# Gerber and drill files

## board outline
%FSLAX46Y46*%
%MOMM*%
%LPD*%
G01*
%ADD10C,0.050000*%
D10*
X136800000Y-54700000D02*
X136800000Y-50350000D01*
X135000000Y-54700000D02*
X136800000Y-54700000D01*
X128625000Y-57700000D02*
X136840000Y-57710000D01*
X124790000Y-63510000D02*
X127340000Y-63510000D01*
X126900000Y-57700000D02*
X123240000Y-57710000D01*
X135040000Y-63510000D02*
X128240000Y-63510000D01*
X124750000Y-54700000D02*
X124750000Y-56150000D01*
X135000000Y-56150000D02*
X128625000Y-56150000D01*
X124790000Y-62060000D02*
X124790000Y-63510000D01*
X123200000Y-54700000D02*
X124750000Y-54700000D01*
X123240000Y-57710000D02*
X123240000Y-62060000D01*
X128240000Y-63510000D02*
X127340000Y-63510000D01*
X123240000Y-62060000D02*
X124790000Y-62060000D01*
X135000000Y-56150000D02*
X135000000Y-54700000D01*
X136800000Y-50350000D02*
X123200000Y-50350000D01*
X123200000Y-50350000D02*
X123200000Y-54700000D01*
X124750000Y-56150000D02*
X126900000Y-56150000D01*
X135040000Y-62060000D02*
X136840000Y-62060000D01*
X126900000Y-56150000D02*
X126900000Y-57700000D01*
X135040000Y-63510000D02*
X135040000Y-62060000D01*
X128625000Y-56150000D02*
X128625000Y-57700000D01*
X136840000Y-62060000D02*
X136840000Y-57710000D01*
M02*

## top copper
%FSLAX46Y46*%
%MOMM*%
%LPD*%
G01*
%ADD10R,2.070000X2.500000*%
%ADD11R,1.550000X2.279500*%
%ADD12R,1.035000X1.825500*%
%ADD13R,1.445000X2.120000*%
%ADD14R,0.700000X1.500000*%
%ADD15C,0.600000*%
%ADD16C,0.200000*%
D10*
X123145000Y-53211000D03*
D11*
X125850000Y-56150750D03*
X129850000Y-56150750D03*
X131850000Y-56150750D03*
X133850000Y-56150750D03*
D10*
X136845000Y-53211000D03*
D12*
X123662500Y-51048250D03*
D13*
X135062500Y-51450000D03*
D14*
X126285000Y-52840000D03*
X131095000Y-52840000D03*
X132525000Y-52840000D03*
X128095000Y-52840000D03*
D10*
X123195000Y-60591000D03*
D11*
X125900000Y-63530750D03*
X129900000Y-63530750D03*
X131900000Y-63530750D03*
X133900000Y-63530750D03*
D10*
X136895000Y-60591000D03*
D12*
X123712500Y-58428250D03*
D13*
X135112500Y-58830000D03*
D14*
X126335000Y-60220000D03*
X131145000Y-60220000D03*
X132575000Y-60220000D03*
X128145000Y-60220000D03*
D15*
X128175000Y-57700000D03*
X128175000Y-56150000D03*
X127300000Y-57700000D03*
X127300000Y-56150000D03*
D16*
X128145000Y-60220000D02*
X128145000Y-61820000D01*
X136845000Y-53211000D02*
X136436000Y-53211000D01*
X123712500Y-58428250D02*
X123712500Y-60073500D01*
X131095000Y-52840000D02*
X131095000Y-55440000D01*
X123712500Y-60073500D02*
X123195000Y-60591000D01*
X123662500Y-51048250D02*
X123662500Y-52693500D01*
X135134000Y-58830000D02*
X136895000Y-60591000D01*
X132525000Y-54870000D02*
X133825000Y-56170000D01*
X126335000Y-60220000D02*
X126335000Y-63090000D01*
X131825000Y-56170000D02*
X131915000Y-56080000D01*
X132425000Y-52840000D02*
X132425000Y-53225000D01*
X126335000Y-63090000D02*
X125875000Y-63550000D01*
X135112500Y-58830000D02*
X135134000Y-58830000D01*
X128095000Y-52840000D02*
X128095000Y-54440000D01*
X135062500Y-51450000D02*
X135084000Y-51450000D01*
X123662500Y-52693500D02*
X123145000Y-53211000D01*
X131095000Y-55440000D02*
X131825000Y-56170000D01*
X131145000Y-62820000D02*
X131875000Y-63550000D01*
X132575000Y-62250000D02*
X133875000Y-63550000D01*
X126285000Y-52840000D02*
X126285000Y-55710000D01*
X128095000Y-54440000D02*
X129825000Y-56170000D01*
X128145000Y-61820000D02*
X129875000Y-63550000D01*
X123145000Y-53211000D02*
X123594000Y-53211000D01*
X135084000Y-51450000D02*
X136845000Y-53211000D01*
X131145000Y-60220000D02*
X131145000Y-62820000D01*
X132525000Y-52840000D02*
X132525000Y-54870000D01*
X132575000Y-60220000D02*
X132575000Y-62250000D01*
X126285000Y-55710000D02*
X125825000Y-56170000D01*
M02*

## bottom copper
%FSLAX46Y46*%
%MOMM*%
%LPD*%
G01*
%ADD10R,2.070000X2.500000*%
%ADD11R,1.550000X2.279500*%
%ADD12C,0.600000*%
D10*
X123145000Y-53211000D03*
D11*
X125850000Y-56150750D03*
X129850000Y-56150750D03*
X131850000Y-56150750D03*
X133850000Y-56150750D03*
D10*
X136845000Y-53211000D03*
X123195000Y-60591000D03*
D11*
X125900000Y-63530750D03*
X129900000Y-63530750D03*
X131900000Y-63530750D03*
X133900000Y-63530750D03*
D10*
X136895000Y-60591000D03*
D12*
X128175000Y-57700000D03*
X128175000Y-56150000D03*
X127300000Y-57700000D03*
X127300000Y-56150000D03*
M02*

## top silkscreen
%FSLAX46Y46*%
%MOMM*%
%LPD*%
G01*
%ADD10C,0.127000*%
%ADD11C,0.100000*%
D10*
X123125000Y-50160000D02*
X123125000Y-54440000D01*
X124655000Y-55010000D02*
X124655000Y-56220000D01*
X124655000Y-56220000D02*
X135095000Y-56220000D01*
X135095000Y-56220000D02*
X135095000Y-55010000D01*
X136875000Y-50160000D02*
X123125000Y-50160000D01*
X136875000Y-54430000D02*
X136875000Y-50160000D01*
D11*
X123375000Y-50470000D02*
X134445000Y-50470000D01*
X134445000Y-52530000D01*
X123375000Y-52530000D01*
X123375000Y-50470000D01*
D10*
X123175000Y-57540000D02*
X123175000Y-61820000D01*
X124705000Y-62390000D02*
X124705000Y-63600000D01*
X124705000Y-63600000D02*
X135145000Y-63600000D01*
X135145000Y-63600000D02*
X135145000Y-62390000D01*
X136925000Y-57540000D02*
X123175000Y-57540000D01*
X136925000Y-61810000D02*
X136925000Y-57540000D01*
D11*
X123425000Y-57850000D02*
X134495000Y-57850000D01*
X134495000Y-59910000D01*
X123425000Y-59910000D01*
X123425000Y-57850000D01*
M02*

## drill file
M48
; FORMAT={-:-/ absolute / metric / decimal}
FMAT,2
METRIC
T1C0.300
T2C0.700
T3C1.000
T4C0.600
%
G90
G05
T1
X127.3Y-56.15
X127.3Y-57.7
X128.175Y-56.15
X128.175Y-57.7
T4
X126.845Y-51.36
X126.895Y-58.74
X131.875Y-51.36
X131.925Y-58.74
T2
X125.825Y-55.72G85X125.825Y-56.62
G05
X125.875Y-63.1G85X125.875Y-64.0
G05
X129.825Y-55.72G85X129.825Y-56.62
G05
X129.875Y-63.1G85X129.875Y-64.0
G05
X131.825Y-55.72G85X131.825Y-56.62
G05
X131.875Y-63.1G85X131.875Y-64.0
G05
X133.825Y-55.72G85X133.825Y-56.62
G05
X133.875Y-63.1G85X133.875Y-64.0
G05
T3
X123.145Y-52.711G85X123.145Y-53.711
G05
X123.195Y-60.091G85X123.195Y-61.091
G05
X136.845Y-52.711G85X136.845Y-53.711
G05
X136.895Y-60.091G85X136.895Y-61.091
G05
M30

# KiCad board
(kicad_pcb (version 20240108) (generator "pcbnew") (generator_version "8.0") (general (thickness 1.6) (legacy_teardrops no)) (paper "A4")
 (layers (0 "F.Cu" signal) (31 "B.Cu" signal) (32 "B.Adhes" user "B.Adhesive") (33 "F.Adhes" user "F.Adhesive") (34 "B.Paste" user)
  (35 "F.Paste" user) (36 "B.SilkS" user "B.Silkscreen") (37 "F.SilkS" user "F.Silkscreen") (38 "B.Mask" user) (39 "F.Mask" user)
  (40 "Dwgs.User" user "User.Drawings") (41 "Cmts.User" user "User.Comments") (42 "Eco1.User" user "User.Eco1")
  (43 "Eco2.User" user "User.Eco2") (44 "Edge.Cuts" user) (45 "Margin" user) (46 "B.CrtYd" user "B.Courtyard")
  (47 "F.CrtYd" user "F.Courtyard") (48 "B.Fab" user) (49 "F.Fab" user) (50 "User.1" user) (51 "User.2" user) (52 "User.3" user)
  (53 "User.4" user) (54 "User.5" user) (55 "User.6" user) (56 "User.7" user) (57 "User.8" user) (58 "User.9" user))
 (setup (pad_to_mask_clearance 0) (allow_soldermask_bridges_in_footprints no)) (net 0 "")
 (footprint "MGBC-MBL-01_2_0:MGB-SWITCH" (layer "F.Cu") (at 129.625 53.97)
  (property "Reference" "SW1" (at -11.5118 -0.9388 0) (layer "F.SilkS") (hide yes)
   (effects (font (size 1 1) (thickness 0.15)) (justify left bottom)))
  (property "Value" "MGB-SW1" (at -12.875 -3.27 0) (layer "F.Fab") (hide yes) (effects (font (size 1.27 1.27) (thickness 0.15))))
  (fp_line (start -6.5 -3.81) (end -6.5 0.47) (stroke (width 0.127) (type solid)) (layer "F.SilkS"))
  (fp_line (start -4.97 1.04) (end -4.97 2.25) (stroke (width 0.127) (type solid)) (layer "F.SilkS"))
  (fp_line (start -4.97 2.25) (end 5.47 2.25) (stroke (width 0.127) (type solid)) (layer "F.SilkS"))
  (fp_line (start 5.47 2.25) (end 5.47 1.04) (stroke (width 0.127) (type solid)) (layer "F.SilkS"))
  (fp_line (start 7.25 -3.81) (end -6.5 -3.81) (stroke (width 0.127) (type solid)) (layer "F.SilkS"))
  (fp_line (start 7.25 0.46) (end 7.25 -3.81) (stroke (width 0.127) (type solid)) (layer "F.SilkS"))
  (fp_rect (start -6.25 -3.5) (end 4.82 -1.44) (stroke (width 0.1) (type default)) (fill none) (layer "F.SilkS"))
  (pad "" np_thru_hole circle (at -2.78 -2.61) (size 0.6 0.6) (drill 0.6) (layers "F&B.Cu" "*.Mask"))
  (pad "" np_thru_hole circle (at 2.25 -2.61) (size 0.6 0.6) (drill 0.6) (layers "F&B.Cu" "*.Mask"))
  (pad "1" thru_hole rect (at -6.48 -0.759) (size 2.07 2.5) (drill oval 1 2) (layers "*.Cu" "*.Mask") (remove_unused_layers no))
  (pad "1" thru_hole rect (at -3.8 2.2) (size 1.55 2.2795) (drill oval 0.7 1.6 (offset 0.025 -0.01925)) (layers "*.Cu" "*.Mask")
   (remove_unused_layers no))
  (pad "1" thru_hole rect (at 0.2 2.2) (size 1.55 2.2795) (drill oval 0.7 1.6 (offset 0.025 -0.01925)) (layers "*.Cu" "*.Mask")
   (remove_unused_layers no))
  (pad "1" thru_hole rect (at 2.2 2.2) (size 1.55 2.2795) (drill oval 0.7 1.6 (offset 0.025 -0.01925)) (layers "*.Cu" "*.Mask")
   (remove_unused_layers no))
  (pad "1" thru_hole rect (at 4.2 2.2) (size 1.55 2.2795) (drill oval 0.7 1.6 (offset 0.025 -0.01925)) (layers "*.Cu" "*.Mask")
   (remove_unused_layers no))
  (pad "1" thru_hole rect (at 7.22 -0.759) (size 2.07 2.5) (drill oval 1 2) (layers "*.Cu" "*.Mask") (remove_unused_layers no))
  (pad "2" smd rect (at -5.9625 -2.92175) (size 1.035 1.8255) (layers "F.Cu" "F.Paste" "F.Mask"))
  (pad "3" smd rect (at 5.4375 -2.52) (size 1.445 2.12) (layers "F.Cu" "F.Paste" "F.Mask"))
  (pad "4" smd rect (at -3.34 -1.13) (size 0.7 1.5) (layers "F.Cu" "F.Paste" "F.Mask"))
  (pad "5" smd rect (at 1.47 -1.13) (size 0.7 1.5) (layers "F.Cu" "F.Paste" "F.Mask"))
  (pad "6" smd rect (at 2.9 -1.13) (size 0.7 1.5) (layers "F.Cu" "F.Paste" "F.Mask"))
  (pad "7" smd rect (at -1.53 -1.13) (size 0.7 1.5) (layers "F.Cu" "F.Paste" "F.Mask")))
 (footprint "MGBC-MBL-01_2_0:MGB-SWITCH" (layer "F.Cu") (at 129.675 61.35)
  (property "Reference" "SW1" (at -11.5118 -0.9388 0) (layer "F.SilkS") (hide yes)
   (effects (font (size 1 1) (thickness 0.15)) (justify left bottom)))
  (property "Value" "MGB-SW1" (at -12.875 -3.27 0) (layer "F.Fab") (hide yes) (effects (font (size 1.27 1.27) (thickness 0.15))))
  (fp_line (start -6.5 -3.81) (end -6.5 0.47) (stroke (width 0.127) (type solid)) (layer "F.SilkS"))
  (fp_line (start -4.97 1.04) (end -4.97 2.25) (stroke (width 0.127) (type solid)) (layer "F.SilkS"))
  (fp_line (start -4.97 2.25) (end 5.47 2.25) (stroke (width 0.127) (type solid)) (layer "F.SilkS"))
  (fp_line (start 5.47 2.25) (end 5.47 1.04) (stroke (width 0.127) (type solid)) (layer "F.SilkS"))
  (fp_line (start 7.25 -3.81) (end -6.5 -3.81) (stroke (width 0.127) (type solid)) (layer "F.SilkS"))
  (fp_line (start 7.25 0.46) (end 7.25 -3.81) (stroke (width 0.127) (type solid)) (layer "F.SilkS"))
  (fp_rect (start -6.25 -3.5) (end 4.82 -1.44) (stroke (width 0.1) (type default)) (fill none) (layer "F.SilkS"))
  (pad "" np_thru_hole circle (at -2.78 -2.61) (size 0.6 0.6) (drill 0.6) (layers "F&B.Cu" "*.Mask"))
  (pad "" np_thru_hole circle (at 2.25 -2.61) (size 0.6 0.6) (drill 0.6) (layers "F&B.Cu" "*.Mask"))
  (pad "1" thru_hole rect (at -6.48 -0.759) (size 2.07 2.5) (drill oval 1 2) (layers "*.Cu" "*.Mask") (remove_unused_layers no))
  (pad "1" thru_hole rect (at -3.8 2.2) (size 1.55 2.2795) (drill oval 0.7 1.6 (offset 0.025 -0.01925)) (layers "*.Cu" "*.Mask")
   (remove_unused_layers no))
  (pad "1" thru_hole rect (at 0.2 2.2) (size 1.55 2.2795) (drill oval 0.7 1.6 (offset 0.025 -0.01925)) (layers "*.Cu" "*.Mask")
   (remove_unused_layers no))
  (pad "1" thru_hole rect (at 2.2 2.2) (size 1.55 2.2795) (drill oval 0.7 1.6 (offset 0.025 -0.01925)) (layers "*.Cu" "*.Mask")
   (remove_unused_layers no))
  (pad "1" thru_hole rect (at 4.2 2.2) (size 1.55 2.2795) (drill oval 0.7 1.6 (offset 0.025 -0.01925)) (layers "*.Cu" "*.Mask")
   (remove_unused_layers no))
  (pad "1" thru_hole rect (at 7.22 -0.759) (size 2.07 2.5) (drill oval 1 2) (layers "*.Cu" "*.Mask") (remove_unused_layers no))
  (pad "2" smd rect (at -5.9625 -2.92175) (size 1.035 1.8255) (layers "F.Cu" "F.Paste" "F.Mask"))
  (pad "3" smd rect (at 5.4375 -2.52) (size 1.445 2.12) (layers "F.Cu" "F.Paste" "F.Mask"))
  (pad "4" smd rect (at -3.34 -1.13) (size 0.7 1.5) (layers "F.Cu" "F.Paste" "F.Mask"))
  (pad "5" smd rect (at 1.47 -1.13) (size 0.7 1.5) (layers "F.Cu" "F.Paste" "F.Mask"))
  (pad "6" smd rect (at 2.9 -1.13) (size 0.7 1.5) (layers "F.Cu" "F.Paste" "F.Mask"))
  (pad "7" smd rect (at -1.53 -1.13) (size 0.7 1.5) (layers "F.Cu" "F.Paste" "F.Mask")))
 (gr_line (start 136.8 54.7) (end 136.8 50.35) (stroke (width 0.05) (type default)) (layer "Edge.Cuts"))
 (gr_line (start 135 54.7) (end 136.8 54.7) (stroke (width 0.05) (type default)) (layer "Edge.Cuts"))
 (gr_line (start 128.625 57.7) (end 136.84 57.71) (stroke (width 0.05) (type default)) (layer "Edge.Cuts"))
 (gr_line (start 124.79 63.51) (end 127.34 63.51) (stroke (width 0.05) (type default)) (layer "Edge.Cuts"))
 (gr_line (start 126.9 57.7) (end 123.24 57.71) (stroke (width 0.05) (type default)) (layer "Edge.Cuts"))
 (gr_line (start 135.04 63.51) (end 128.24 63.51) (stroke (width 0.05) (type default)) (layer "Edge.Cuts"))
 (gr_line (start 124.75 54.7) (end 124.75 56.15) (stroke (width 0.05) (type default)) (layer "Edge.Cuts"))
 (gr_line (start 135 56.15) (end 128.625 56.15) (stroke (width 0.05) (type default)) (layer "Edge.Cuts"))
 (gr_line (start 124.79 62.06) (end 124.79 63.51) (stroke (width 0.05) (type default)) (layer "Edge.Cuts"))
 (gr_line (start 123.2 54.7) (end 124.75 54.7) (stroke (width 0.05) (type default)) (layer "Edge.Cuts"))
 (gr_line (start 123.24 57.71) (end 123.24 62.06) (stroke (width 0.05) (type default)) (layer "Edge.Cuts"))
 (gr_line (start 128.24 63.51) (end 127.34 63.51) (stroke (width 0.05) (type default)) (layer "Edge.Cuts"))
 (gr_line (start 123.24 62.06) (end 124.79 62.06) (stroke (width 0.05) (type default)) (layer "Edge.Cuts"))
 (gr_line (start 135 56.15) (end 135 54.7) (stroke (width 0.05) (type default)) (layer "Edge.Cuts"))
 (gr_line (start 136.8 50.35) (end 123.2 50.35) (stroke (width 0.05) (type default)) (layer "Edge.Cuts"))
 (gr_line (start 123.2 50.35) (end 123.2 54.7) (stroke (width 0.05) (type default)) (layer "Edge.Cuts"))
 (gr_line (start 124.75 56.15) (end 126.9 56.15) (stroke (width 0.05) (type default)) (layer "Edge.Cuts"))
 (gr_line (start 135.04 62.06) (end 136.84 62.06) (stroke (width 0.05) (type default)) (layer "Edge.Cuts"))
 (gr_line (start 126.9 56.15) (end 126.9 57.7) (stroke (width 0.05) (type default)) (layer "Edge.Cuts"))
 (gr_line (start 135.04 63.51) (end 135.04 62.06) (stroke (width 0.05) (type default)) (layer "Edge.Cuts"))
 (gr_line (start 128.625 56.15) (end 128.625 57.7) (stroke (width 0.05) (type default)) (layer "Edge.Cuts"))
 (gr_line (start 136.84 62.06) (end 136.84 57.71) (stroke (width 0.05) (type default)) (layer "Edge.Cuts"))
 (segment (start 128.145 60.22) (end 128.145 61.82) (width 0.2) (layer "F.Cu") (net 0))
 (segment (start 136.845 53.211) (end 136.436 53.211) (width 0.2) (layer "F.Cu") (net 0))
 (segment (start 123.7125 58.42825) (end 123.7125 60.0735) (width 0.2) (layer "F.Cu") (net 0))
 (segment (start 131.095 52.84) (end 131.095 55.44) (width 0.2) (layer "F.Cu") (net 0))
 (segment (start 123.7125 60.0735) (end 123.195 60.591) (width 0.2) (layer "F.Cu") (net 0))
 (segment (start 123.6625 51.04825) (end 123.6625 52.6935) (width 0.2) (layer "F.Cu") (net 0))
 (segment (start 135.134 58.83) (end 136.895 60.591) (width 0.2) (layer "F.Cu") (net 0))
 (segment (start 132.525 54.87) (end 133.825 56.17) (width 0.2) (layer "F.Cu") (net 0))
 (segment (start 126.335 60.22) (end 126.335 63.09) (width 0.2) (layer "F.Cu") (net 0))
 (segment (start 131.825 56.17) (end 131.915 56.08) (width 0.2) (layer "F.Cu") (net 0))
 (segment (start 132.425 52.84) (end 132.425 53.225) (width 0.2) (layer "F.Cu") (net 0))
 (segment (start 126.335 63.09) (end 125.875 63.55) (width 0.2) (layer "F.Cu") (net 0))
 (segment (start 135.1125 58.83) (end 135.134 58.83) (width 0.2) (layer "F.Cu") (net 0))
 (segment (start 128.095 52.84) (end 128.095 54.44) (width 0.2) (layer "F.Cu") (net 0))
 (segment (start 135.0625 51.45) (end 135.084 51.45) (width 0.2) (layer "F.Cu") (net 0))
 (segment (start 123.6625 52.6935) (end 123.145 53.211) (width 0.2) (layer "F.Cu") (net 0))
 (segment (start 131.095 55.44) (end 131.825 56.17) (width 0.2) (layer "F.Cu") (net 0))
 (segment (start 131.145 62.82) (end 131.875 63.55) (width 0.2) (layer "F.Cu") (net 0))
 (segment (start 132.575 62.25) (end 133.875 63.55) (width 0.2) (layer "F.Cu") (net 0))
 (segment (start 126.285 52.84) (end 126.285 55.71) (width 0.2) (layer "F.Cu") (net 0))
 (segment (start 128.095 54.44) (end 129.825 56.17) (width 0.2) (layer "F.Cu") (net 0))
 (segment (start 128.145 61.82) (end 129.875 63.55) (width 0.2) (layer "F.Cu") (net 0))
 (segment (start 123.145 53.211) (end 123.594 53.211) (width 0.2) (layer "F.Cu") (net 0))
 (segment (start 135.084 51.45) (end 136.845 53.211) (width 0.2) (layer "F.Cu") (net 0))
 (segment (start 131.145 60.22) (end 131.145 62.82) (width 0.2) (layer "F.Cu") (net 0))
 (segment (start 132.525 52.84) (end 132.525 54.87) (width 0.2) (layer "F.Cu") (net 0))
 (segment (start 132.575 60.22) (end 132.575 62.25) (width 0.2) (layer "F.Cu") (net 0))
 (segment (start 126.285 55.71) (end 125.825 56.17) (width 0.2) (layer "F.Cu") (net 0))
 (via (at 128.175 57.7) (size 0.6) (drill 0.3) (layers "F.Cu" "B.Cu") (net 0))
 (via (at 128.175 56.15) (size 0.6) (drill 0.3) (layers "F.Cu" "B.Cu") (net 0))
 (via (at 127.3 57.7) (size 0.6) (drill 0.3) (layers "F.Cu" "B.Cu") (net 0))
 (via (at 127.3 56.15) (size 0.6) (drill 0.3) (layers "F.Cu" "B.Cu") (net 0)))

